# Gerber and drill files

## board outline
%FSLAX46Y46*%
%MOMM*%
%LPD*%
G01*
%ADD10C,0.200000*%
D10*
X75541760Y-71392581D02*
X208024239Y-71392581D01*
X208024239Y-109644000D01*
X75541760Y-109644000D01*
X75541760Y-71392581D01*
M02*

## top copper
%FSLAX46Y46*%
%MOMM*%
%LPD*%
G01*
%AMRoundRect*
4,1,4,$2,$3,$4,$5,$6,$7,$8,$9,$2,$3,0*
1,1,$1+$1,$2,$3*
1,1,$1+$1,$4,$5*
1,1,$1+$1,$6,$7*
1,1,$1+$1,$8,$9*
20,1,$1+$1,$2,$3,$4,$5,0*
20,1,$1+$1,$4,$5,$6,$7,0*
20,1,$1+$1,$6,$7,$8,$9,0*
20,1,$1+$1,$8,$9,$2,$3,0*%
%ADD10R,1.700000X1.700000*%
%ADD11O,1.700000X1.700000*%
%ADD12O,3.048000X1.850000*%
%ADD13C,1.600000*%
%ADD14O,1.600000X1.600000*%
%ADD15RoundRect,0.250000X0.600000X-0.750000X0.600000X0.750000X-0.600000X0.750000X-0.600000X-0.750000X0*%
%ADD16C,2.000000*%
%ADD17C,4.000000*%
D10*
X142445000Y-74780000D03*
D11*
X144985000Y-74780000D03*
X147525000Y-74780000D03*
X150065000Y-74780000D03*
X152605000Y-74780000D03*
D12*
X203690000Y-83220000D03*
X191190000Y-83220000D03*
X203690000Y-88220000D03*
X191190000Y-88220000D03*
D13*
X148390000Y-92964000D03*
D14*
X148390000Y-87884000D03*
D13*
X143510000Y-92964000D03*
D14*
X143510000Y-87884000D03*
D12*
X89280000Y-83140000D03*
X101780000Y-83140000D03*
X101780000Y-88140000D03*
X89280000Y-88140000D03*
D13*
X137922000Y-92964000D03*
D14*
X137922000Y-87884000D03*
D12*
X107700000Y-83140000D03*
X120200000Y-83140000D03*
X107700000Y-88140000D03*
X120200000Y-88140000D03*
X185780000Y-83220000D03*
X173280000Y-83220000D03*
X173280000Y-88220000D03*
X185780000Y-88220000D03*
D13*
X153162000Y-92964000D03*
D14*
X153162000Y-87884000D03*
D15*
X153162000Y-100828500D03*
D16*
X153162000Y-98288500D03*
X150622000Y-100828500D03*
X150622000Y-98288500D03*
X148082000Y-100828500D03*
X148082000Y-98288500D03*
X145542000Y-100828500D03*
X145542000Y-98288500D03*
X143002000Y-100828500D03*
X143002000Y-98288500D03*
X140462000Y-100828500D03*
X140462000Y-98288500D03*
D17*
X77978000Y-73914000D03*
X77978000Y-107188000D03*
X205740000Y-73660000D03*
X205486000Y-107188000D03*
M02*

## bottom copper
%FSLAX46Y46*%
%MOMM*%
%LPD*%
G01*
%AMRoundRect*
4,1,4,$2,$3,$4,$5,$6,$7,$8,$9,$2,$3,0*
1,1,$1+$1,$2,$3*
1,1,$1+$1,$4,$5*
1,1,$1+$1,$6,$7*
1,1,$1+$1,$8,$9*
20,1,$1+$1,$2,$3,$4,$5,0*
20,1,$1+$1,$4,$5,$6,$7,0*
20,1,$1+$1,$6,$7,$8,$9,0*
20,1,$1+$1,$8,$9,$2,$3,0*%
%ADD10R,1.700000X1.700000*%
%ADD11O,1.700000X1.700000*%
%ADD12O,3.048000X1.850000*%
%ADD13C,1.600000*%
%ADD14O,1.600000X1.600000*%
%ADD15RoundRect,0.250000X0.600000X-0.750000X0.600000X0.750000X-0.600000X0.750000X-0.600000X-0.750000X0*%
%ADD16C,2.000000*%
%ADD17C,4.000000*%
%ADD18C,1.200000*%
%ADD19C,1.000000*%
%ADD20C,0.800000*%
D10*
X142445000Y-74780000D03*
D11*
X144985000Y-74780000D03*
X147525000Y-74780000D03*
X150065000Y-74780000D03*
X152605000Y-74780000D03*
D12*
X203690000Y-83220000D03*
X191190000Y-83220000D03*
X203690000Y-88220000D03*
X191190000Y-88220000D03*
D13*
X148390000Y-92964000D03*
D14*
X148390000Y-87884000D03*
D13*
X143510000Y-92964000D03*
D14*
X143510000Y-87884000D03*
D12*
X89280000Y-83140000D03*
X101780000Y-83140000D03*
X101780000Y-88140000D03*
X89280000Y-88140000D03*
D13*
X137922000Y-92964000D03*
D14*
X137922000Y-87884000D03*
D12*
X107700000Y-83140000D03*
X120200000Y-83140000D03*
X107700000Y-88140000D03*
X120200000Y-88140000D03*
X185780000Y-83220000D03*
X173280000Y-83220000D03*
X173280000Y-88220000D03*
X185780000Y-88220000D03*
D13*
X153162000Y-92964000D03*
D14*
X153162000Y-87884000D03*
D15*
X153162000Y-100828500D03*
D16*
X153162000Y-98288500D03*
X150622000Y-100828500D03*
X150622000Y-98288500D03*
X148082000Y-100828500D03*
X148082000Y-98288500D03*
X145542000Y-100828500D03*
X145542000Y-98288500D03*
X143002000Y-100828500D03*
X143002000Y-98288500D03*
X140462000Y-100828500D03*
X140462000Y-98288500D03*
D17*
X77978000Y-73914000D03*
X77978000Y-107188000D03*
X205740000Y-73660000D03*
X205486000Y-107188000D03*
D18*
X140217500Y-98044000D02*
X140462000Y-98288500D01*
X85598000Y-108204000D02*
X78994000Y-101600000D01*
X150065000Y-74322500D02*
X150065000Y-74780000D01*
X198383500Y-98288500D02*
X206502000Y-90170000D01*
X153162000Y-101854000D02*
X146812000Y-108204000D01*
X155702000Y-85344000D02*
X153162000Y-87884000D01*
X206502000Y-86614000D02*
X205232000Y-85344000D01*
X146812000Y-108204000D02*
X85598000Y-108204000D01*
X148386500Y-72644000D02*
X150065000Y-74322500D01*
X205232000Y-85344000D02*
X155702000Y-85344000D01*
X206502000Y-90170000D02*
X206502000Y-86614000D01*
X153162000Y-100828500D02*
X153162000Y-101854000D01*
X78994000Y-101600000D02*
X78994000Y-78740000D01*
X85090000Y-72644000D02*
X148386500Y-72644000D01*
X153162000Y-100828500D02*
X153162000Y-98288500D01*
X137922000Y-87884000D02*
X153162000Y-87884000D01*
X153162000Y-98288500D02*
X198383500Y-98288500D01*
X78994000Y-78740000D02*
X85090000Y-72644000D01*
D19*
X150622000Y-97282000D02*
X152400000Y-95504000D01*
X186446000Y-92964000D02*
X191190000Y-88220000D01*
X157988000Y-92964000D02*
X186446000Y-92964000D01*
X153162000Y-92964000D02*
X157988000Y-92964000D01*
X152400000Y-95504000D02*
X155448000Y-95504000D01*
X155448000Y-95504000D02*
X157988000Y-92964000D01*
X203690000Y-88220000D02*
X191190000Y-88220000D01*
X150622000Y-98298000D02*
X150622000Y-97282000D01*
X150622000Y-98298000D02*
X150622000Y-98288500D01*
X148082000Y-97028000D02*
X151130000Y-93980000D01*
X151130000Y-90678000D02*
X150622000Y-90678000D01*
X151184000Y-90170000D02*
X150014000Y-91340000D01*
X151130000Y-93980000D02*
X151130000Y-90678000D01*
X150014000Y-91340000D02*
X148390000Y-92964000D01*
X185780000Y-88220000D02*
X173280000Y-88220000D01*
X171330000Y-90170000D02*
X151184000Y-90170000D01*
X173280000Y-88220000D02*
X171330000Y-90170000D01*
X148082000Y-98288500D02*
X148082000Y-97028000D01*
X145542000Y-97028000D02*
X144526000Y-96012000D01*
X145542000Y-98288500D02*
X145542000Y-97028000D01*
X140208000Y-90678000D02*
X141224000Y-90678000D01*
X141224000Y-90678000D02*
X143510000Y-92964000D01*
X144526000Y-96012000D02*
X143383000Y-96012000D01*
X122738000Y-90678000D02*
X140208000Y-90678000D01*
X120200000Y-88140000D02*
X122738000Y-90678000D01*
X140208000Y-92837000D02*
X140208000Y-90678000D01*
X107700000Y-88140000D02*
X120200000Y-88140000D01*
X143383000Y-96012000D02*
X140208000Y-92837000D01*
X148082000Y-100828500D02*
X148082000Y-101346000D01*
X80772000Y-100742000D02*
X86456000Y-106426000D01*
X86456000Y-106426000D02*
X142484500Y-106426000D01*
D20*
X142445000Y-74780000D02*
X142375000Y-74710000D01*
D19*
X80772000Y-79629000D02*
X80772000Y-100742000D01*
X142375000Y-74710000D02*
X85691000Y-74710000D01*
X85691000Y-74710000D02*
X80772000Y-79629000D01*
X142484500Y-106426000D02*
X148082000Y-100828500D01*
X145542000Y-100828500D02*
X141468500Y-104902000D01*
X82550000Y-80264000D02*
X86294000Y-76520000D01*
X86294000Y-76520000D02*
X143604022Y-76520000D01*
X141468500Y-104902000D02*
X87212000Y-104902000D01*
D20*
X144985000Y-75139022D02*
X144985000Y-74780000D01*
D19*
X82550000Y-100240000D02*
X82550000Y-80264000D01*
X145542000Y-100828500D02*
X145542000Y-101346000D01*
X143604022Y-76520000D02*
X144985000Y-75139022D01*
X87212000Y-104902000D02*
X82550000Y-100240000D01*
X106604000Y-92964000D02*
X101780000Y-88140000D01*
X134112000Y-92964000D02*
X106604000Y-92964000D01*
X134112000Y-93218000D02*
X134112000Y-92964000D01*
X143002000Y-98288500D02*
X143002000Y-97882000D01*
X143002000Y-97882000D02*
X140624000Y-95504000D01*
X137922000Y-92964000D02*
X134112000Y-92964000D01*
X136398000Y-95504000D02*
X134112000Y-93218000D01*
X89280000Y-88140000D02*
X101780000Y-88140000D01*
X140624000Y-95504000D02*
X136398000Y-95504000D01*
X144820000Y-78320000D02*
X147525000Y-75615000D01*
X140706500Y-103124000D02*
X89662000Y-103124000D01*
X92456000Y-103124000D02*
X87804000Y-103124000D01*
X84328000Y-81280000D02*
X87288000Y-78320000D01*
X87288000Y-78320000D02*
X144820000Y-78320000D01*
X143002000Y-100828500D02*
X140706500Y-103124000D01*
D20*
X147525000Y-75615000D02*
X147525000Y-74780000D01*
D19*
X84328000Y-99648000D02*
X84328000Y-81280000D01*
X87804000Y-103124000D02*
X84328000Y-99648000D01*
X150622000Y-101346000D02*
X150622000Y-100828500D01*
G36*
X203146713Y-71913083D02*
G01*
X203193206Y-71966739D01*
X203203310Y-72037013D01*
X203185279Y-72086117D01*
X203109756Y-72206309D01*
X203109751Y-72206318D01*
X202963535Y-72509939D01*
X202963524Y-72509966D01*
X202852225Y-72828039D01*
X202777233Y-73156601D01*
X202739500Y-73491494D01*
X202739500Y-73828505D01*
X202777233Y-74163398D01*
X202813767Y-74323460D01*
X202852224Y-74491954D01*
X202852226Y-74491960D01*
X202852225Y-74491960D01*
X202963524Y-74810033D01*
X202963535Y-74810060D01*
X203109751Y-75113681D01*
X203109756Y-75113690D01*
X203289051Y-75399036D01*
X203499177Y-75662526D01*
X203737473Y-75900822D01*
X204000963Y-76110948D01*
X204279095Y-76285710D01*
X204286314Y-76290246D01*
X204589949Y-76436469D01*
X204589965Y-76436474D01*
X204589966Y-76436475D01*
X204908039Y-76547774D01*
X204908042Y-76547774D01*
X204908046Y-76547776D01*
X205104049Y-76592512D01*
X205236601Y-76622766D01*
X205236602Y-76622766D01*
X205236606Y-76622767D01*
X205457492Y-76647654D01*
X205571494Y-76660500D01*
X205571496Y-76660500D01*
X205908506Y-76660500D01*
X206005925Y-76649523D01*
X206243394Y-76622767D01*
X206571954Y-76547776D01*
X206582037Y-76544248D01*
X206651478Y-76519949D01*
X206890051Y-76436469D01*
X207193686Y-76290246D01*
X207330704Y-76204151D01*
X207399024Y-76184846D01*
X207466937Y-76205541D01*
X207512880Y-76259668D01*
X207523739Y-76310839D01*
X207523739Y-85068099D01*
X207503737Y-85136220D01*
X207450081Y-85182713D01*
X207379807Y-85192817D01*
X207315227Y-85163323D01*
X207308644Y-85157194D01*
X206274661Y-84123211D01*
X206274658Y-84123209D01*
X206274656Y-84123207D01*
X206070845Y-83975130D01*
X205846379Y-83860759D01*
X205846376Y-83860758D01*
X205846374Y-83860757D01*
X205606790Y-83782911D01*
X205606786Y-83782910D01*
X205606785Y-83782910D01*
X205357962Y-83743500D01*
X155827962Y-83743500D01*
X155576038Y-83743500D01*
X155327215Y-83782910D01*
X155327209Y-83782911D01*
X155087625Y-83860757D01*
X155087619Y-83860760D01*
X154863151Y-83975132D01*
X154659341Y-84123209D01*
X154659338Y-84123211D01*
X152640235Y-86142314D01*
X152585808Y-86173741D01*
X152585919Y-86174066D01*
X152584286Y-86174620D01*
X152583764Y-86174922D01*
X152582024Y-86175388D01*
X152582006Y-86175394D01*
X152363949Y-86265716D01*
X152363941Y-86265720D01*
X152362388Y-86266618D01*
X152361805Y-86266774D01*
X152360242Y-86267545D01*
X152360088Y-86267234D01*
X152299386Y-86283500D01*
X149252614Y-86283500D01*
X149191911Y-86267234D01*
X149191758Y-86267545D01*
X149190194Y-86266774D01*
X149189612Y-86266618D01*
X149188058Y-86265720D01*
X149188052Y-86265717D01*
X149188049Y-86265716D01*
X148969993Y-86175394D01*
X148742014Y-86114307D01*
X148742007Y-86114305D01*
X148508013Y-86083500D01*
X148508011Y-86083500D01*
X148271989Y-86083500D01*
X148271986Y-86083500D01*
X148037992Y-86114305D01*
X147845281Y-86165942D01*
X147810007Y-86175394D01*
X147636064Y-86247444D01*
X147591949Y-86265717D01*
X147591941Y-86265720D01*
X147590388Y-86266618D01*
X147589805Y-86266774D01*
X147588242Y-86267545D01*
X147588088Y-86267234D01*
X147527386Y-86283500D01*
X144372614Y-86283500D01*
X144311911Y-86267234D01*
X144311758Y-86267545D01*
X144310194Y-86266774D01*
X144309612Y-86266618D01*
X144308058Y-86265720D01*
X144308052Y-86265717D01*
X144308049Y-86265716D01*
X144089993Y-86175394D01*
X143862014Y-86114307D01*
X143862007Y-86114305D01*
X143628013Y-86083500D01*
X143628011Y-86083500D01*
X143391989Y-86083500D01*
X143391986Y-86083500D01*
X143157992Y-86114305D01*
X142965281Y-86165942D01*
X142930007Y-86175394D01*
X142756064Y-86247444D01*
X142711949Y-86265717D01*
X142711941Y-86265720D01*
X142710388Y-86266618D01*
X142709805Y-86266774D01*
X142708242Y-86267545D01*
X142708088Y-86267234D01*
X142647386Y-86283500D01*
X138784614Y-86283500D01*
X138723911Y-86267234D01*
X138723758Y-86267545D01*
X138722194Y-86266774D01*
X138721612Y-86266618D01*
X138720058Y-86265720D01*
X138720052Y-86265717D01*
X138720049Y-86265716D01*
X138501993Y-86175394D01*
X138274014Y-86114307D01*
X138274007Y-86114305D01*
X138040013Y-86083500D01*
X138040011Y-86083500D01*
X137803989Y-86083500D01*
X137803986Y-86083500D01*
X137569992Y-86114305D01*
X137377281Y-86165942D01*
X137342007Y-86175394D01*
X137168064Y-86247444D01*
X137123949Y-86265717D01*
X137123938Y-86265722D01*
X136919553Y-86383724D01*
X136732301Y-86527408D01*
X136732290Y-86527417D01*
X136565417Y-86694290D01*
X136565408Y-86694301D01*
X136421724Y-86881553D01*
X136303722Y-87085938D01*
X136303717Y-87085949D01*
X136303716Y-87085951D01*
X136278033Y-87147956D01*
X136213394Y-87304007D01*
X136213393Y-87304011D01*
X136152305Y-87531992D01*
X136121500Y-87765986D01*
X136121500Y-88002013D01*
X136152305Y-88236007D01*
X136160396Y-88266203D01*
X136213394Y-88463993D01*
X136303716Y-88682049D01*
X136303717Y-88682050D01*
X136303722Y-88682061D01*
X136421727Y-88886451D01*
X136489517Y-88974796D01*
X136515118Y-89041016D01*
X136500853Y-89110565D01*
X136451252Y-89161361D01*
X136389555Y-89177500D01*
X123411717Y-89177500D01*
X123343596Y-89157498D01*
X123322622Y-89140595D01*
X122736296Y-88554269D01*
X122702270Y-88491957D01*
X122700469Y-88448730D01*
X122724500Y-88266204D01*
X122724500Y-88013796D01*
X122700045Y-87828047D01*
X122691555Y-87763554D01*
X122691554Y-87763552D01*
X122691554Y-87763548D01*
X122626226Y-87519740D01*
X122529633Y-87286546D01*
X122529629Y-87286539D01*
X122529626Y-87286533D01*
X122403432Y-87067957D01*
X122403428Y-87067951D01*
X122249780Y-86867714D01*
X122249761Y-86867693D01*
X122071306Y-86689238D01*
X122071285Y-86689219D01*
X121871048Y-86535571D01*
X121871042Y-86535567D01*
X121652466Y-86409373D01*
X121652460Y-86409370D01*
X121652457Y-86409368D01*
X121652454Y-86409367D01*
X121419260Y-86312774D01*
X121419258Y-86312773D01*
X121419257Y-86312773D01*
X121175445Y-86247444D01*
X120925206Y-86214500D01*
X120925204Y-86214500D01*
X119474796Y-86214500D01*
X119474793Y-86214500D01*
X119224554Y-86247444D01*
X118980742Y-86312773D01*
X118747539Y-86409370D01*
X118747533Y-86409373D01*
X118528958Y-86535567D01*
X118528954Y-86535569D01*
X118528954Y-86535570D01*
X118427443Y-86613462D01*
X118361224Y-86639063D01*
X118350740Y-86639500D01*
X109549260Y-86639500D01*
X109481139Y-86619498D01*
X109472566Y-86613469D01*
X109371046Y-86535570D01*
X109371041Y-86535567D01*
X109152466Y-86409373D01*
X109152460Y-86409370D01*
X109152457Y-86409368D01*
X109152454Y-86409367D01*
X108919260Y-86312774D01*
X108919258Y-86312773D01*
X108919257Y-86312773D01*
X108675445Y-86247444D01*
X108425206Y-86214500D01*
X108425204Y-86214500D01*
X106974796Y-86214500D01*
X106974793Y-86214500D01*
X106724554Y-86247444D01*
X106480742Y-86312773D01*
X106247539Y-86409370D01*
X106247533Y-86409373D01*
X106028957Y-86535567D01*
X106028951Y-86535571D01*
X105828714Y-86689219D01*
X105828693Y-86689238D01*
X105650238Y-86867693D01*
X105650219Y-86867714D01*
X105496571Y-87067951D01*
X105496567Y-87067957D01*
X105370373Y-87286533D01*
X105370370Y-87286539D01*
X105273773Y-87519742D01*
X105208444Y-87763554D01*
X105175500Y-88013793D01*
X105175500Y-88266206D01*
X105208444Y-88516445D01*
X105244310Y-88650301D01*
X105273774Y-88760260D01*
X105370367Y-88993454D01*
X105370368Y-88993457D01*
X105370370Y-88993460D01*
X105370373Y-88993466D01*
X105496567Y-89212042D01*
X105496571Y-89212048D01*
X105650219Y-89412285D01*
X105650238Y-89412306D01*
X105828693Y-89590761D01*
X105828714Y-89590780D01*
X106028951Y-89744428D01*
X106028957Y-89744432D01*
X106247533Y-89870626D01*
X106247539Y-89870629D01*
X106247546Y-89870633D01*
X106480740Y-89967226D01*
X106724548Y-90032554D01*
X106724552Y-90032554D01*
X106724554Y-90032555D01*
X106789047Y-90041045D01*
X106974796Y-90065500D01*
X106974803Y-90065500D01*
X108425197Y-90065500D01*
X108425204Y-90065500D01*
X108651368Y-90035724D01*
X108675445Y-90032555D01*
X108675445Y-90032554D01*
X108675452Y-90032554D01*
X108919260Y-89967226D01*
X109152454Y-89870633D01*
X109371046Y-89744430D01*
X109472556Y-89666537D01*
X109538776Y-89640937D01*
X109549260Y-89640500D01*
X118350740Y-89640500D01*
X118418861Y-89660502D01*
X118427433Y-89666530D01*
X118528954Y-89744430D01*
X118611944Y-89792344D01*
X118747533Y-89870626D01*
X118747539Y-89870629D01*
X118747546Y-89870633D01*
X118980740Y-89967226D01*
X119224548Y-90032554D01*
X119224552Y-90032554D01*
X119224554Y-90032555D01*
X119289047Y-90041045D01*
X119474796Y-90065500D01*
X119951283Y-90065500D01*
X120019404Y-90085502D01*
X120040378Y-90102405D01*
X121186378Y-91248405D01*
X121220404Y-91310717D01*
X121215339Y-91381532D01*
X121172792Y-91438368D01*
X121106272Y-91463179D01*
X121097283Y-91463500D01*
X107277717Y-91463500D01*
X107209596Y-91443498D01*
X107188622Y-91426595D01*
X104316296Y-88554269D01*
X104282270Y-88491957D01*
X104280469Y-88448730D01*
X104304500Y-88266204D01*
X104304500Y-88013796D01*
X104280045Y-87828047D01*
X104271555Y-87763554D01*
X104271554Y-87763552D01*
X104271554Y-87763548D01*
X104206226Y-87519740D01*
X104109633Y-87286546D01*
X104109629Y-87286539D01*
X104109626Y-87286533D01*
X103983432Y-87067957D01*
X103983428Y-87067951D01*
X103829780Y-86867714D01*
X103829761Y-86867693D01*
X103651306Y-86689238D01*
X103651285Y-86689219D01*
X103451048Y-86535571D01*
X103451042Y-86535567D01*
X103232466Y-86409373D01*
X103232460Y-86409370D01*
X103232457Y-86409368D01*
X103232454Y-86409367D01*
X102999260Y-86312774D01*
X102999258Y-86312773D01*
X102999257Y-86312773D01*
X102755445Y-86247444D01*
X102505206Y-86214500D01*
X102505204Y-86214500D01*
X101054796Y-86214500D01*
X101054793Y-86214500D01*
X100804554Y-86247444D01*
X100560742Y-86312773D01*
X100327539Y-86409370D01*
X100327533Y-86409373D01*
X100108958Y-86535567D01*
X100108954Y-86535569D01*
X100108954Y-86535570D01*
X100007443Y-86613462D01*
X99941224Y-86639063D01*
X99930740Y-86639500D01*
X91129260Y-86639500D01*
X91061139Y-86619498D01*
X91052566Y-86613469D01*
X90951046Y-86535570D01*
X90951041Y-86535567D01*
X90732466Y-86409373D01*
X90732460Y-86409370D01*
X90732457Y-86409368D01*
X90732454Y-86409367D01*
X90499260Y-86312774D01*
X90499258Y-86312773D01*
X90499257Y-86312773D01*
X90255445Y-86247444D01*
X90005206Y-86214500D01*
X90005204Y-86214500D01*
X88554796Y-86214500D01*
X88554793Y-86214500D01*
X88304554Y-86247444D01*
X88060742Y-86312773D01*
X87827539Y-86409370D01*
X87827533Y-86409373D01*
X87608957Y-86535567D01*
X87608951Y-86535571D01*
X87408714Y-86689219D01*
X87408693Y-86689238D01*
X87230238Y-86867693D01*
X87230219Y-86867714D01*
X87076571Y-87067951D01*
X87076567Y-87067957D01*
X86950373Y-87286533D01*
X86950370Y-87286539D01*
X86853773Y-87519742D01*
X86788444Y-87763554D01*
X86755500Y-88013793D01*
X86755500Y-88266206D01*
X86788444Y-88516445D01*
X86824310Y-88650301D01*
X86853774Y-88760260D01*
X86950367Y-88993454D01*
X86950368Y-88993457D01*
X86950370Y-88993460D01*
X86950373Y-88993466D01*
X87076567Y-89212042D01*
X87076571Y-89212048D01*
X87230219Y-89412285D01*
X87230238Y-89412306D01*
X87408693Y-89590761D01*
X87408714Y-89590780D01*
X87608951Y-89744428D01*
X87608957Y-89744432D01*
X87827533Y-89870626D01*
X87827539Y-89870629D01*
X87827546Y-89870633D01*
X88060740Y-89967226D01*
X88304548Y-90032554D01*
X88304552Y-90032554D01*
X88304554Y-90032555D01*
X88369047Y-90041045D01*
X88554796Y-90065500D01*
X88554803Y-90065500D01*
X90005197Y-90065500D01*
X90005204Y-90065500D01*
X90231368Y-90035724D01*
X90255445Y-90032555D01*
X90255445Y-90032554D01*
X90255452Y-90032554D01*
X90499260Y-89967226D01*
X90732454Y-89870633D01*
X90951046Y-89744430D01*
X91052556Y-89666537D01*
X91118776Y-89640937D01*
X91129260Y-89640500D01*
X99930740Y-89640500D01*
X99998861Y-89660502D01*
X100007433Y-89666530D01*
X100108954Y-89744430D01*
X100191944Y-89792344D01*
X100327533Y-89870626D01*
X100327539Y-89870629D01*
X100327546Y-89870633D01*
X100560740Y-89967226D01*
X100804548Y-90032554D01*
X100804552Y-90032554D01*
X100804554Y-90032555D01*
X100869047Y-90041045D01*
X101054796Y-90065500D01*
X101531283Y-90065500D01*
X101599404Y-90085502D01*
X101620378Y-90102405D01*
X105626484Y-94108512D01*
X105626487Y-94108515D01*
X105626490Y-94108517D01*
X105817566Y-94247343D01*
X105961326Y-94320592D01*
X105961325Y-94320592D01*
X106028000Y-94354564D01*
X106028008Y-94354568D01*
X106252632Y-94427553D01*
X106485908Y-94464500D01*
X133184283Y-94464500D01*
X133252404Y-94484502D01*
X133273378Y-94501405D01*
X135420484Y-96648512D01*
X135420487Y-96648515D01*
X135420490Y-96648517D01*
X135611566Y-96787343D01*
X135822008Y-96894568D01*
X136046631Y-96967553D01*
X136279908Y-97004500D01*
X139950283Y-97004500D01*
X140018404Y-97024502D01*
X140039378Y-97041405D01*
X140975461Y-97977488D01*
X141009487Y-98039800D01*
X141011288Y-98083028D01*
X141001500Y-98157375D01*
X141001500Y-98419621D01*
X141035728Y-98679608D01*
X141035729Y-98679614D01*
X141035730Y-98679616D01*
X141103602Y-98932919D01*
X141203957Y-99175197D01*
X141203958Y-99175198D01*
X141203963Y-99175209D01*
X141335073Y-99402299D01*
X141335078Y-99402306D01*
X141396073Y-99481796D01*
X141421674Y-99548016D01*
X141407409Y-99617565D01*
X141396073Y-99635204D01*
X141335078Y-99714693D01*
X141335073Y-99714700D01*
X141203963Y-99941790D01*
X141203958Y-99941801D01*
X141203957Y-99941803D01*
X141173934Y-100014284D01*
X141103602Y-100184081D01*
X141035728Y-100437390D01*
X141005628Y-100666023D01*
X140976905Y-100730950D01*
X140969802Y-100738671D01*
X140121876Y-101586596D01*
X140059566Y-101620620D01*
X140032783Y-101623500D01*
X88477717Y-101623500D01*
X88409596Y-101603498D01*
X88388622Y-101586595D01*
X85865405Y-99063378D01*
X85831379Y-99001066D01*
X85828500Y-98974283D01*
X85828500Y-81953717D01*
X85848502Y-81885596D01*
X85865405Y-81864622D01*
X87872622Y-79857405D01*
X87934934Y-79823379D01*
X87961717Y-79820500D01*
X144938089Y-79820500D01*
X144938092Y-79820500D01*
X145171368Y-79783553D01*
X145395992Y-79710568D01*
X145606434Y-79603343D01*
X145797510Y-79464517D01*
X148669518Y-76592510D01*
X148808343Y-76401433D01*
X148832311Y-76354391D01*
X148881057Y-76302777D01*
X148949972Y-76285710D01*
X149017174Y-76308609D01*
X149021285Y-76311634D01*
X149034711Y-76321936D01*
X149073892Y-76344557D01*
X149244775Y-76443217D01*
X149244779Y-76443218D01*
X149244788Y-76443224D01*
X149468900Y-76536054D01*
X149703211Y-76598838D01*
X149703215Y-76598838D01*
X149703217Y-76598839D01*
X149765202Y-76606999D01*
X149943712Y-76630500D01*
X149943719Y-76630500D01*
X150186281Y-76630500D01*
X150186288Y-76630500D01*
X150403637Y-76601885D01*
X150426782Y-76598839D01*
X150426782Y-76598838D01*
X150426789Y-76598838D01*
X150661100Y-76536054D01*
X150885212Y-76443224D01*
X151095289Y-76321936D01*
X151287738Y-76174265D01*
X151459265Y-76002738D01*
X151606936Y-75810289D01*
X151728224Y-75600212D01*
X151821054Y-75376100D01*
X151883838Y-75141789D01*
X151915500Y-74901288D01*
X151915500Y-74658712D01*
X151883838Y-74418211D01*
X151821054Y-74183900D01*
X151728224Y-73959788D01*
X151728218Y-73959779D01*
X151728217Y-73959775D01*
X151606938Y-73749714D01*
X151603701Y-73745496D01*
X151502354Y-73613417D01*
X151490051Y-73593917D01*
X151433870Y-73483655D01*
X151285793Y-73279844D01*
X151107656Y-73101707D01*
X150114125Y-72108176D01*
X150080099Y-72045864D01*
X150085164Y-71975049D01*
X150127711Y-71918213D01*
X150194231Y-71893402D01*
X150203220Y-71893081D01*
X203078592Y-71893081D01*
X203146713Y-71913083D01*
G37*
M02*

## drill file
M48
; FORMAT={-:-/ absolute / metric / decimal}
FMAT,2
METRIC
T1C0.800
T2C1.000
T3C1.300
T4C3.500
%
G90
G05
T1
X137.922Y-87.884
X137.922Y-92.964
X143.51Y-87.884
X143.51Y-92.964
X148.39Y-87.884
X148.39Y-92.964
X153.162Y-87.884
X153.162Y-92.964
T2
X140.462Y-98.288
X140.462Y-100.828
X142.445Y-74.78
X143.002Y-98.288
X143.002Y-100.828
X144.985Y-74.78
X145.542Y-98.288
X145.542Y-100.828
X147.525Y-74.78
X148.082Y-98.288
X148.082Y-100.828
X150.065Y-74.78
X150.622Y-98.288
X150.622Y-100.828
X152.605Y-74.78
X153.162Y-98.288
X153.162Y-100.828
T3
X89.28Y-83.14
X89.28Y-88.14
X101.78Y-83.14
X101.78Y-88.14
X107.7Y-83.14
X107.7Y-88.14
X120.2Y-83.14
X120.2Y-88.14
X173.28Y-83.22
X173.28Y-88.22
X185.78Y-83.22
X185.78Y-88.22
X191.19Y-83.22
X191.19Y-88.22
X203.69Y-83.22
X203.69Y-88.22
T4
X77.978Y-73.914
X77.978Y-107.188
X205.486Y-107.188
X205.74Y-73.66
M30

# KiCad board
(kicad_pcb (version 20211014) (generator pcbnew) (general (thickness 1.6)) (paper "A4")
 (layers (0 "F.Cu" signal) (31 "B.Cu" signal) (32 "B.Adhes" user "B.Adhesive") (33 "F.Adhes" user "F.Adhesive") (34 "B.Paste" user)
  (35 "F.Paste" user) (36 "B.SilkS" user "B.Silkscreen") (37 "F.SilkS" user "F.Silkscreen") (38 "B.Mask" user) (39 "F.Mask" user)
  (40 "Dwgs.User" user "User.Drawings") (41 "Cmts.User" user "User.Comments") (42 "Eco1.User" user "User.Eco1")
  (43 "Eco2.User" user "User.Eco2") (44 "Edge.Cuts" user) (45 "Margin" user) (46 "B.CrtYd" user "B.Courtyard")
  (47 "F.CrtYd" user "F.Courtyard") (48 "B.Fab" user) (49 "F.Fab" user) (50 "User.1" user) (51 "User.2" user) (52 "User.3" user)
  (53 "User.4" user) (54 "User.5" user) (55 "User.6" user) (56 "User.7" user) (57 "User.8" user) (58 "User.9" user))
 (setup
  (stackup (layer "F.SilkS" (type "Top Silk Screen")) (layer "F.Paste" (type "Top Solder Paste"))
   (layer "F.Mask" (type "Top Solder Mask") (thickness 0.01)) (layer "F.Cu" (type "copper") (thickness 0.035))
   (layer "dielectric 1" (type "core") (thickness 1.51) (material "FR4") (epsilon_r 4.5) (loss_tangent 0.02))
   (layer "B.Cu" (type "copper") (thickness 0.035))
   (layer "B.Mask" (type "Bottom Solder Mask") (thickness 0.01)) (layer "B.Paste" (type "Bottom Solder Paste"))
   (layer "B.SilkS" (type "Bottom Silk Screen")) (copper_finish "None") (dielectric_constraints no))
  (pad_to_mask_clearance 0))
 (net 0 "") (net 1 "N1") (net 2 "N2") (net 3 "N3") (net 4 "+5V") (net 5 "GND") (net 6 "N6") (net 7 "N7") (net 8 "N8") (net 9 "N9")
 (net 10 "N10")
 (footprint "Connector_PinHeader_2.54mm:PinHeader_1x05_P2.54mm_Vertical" (layer "F.Cu") (at 142.445 74.78 90)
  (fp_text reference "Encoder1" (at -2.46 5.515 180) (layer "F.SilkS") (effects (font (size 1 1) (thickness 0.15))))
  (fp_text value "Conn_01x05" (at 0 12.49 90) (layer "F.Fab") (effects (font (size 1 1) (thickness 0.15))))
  (pad "1" thru_hole rect (at 0 0 90) (size 1.7 1.7) (drill 1) (layers *.Cu *.Mask) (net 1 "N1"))
  (pad "2" thru_hole oval (at 0 2.54 90) (size 1.7 1.7) (drill 1) (layers *.Cu *.Mask) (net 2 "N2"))
  (pad "3" thru_hole oval (at 0 5.08 90) (size 1.7 1.7) (drill 1) (layers *.Cu *.Mask) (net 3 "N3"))
  (pad "4" thru_hole oval (at 0 7.62 90) (size 1.7 1.7) (drill 1) (layers *.Cu *.Mask) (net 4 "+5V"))
  (pad "5" thru_hole oval (at 0 10.16 90) (size 1.7 1.7) (drill 1) (layers *.Cu *.Mask) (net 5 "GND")))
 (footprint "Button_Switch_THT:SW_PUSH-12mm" (layer "F.Cu") (at 191.19 83.22)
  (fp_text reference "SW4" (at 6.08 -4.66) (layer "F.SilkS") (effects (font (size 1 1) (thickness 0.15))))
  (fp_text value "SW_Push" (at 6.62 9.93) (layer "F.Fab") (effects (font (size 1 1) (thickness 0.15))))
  (pad "1" thru_hole oval (at 12.5 0) (size 3.048 1.85) (drill 1.3) (layers *.Cu *.Mask) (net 5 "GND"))
  (pad "1" thru_hole oval (at 0 0) (size 3.048 1.85) (drill 1.3) (layers *.Cu *.Mask) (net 5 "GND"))
  (pad "2" thru_hole oval (at 12.5 5) (size 3.048 1.85) (drill 1.3) (layers *.Cu *.Mask) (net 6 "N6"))
  (pad "2" thru_hole oval (at 0 5) (size 3.048 1.85) (drill 1.3) (layers *.Cu *.Mask) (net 6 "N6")))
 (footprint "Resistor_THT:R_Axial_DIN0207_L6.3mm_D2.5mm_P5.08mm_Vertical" (layer "F.Cu") (at 148.39 92.964 90)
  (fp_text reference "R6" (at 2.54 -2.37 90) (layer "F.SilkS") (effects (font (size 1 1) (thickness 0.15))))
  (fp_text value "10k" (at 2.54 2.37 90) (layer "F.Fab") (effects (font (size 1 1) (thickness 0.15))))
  (pad "1" thru_hole circle (at 0 0 90) (size 1.6 1.6) (drill 0.8) (layers *.Cu *.Mask) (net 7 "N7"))
  (pad "2" thru_hole oval (at 5.08 0 90) (size 1.6 1.6) (drill 0.8) (layers *.Cu *.Mask) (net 4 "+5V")))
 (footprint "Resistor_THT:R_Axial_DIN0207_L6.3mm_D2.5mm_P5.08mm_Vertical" (layer "F.Cu") (at 143.51 92.964 90)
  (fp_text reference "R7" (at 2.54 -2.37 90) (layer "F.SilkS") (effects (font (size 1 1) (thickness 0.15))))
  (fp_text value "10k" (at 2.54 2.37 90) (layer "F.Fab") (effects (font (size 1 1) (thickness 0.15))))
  (pad "1" thru_hole circle (at 0 0 90) (size 1.6 1.6) (drill 0.8) (layers *.Cu *.Mask) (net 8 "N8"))
  (pad "2" thru_hole oval (at 5.08 0 90) (size 1.6 1.6) (drill 0.8) (layers *.Cu *.Mask) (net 4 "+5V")))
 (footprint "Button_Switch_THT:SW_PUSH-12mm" (layer "F.Cu") (at 89.28 83.14)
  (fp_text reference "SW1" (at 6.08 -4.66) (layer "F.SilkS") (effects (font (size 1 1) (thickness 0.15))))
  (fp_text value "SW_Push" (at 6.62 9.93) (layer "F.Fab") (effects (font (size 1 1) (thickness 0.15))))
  (pad "1" thru_hole oval (at 0 0) (size 3.048 1.85) (drill 1.3) (layers *.Cu *.Mask) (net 5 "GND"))
  (pad "1" thru_hole oval (at 12.5 0) (size 3.048 1.85) (drill 1.3) (layers *.Cu *.Mask) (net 5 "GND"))
  (pad "2" thru_hole oval (at 12.5 5) (size 3.048 1.85) (drill 1.3) (layers *.Cu *.Mask) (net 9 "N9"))
  (pad "2" thru_hole oval (at 0 5) (size 3.048 1.85) (drill 1.3) (layers *.Cu *.Mask) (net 9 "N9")))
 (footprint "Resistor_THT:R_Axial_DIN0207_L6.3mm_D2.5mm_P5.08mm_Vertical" (layer "F.Cu") (at 137.922 92.964 90)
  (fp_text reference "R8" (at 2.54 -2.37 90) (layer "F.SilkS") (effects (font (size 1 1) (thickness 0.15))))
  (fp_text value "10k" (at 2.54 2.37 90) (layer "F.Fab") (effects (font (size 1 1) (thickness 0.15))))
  (pad "1" thru_hole circle (at 0 0 90) (size 1.6 1.6) (drill 0.8) (layers *.Cu *.Mask) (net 9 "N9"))
  (pad "2" thru_hole oval (at 5.08 0 90) (size 1.6 1.6) (drill 0.8) (layers *.Cu *.Mask) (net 4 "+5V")))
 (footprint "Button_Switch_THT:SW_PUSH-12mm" (layer "F.Cu") (at 107.7 83.14)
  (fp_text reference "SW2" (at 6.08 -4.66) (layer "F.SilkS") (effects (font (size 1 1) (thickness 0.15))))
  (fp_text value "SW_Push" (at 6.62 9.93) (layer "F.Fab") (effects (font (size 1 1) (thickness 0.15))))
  (pad "1" thru_hole oval (at 0 0) (size 3.048 1.85) (drill 1.3) (layers *.Cu *.Mask) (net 5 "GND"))
  (pad "1" thru_hole oval (at 12.5 0) (size 3.048 1.85) (drill 1.3) (layers *.Cu *.Mask) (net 5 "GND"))
  (pad "2" thru_hole oval (at 0 5) (size 3.048 1.85) (drill 1.3) (layers *.Cu *.Mask) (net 8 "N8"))
  (pad "2" thru_hole oval (at 12.5 5) (size 3.048 1.85) (drill 1.3) (layers *.Cu *.Mask) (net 8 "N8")))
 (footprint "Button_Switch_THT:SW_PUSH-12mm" (layer "F.Cu") (at 173.28 83.22)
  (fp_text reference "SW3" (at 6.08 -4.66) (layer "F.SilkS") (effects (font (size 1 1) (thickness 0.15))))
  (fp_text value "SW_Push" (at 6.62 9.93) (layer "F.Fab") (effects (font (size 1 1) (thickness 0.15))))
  (pad "1" thru_hole oval (at 12.5 0) (size 3.048 1.85) (drill 1.3) (layers *.Cu *.Mask) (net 5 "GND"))
  (pad "1" thru_hole oval (at 0 0) (size 3.048 1.85) (drill 1.3) (layers *.Cu *.Mask) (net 5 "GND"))
  (pad "2" thru_hole oval (at 0 5) (size 3.048 1.85) (drill 1.3) (layers *.Cu *.Mask) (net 7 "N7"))
  (pad "2" thru_hole oval (at 12.5 5) (size 3.048 1.85) (drill 1.3) (layers *.Cu *.Mask) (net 7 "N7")))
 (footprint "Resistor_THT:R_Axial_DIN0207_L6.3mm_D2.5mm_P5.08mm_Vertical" (layer "F.Cu") (at 153.162 92.964 90)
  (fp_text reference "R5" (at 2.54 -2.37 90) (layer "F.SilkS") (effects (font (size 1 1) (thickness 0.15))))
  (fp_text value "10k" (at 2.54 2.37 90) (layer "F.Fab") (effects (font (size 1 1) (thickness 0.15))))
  (pad "1" thru_hole circle (at 0 0 90) (size 1.6 1.6) (drill 0.8) (layers *.Cu *.Mask) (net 6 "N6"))
  (pad "2" thru_hole oval (at 5.08 0 90) (size 1.6 1.6) (drill 0.8) (layers *.Cu *.Mask) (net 4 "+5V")))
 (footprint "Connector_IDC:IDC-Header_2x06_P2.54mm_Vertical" (layer "B.Cu") (at 153.162 100.8285 90)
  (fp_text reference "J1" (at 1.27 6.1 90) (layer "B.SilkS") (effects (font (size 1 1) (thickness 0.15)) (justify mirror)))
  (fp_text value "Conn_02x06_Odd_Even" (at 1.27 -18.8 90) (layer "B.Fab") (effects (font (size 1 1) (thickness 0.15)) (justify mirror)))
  (pad "1" thru_hole roundrect (at 0 0 90) (size 2 1.7) (drill 1) (layers *.Cu *.Mask) (roundrect_rratio 0.147059) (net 4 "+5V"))
  (pad "2" thru_hole circle (at 2.54 0 90) (size 2 2) (drill 1) (layers *.Cu *.Mask) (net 4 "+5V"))
  (pad "3" thru_hole circle (at 0 -2.54 90) (size 2 2) (drill 1) (layers *.Cu *.Mask) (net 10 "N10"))
  (pad "4" thru_hole circle (at 2.54 -2.54 90) (size 2 2) (drill 1) (layers *.Cu *.Mask) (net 6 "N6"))
  (pad "5" thru_hole circle (at 0 -5.08 90) (size 2 2) (drill 1) (layers *.Cu *.Mask) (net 1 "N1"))
  (pad "6" thru_hole circle (at 2.54 -5.08 90) (size 2 2) (drill 1) (layers *.Cu *.Mask) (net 7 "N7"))
  (pad "7" thru_hole circle (at 0 -7.62 90) (size 2 2) (drill 1) (layers *.Cu *.Mask) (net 2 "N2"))
  (pad "8" thru_hole circle (at 2.54 -7.62 90) (size 2 2) (drill 1) (layers *.Cu *.Mask) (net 8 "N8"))
  (pad "9" thru_hole circle (at 0 -10.16 90) (size 2 2) (drill 1) (layers *.Cu *.Mask) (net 3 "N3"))
  (pad "10" thru_hole circle (at 2.54 -10.16 90) (size 2 2) (drill 1) (layers *.Cu *.Mask) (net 9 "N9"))
  (pad "11" thru_hole circle (at 0 -12.7 90) (size 2 2) (drill 1) (layers *.Cu *.Mask) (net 5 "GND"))
  (pad "12" thru_hole circle (at 2.54 -12.7 90) (size 2 2) (drill 1) (layers *.Cu *.Mask) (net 5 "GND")))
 (gr_rect (start 75.54176 71.392581) (end 208.024239 109.644) (layer "Edge.Cuts") (width 0.2) (fill none))
 (via (at 77.978 73.914) (size 4) (drill 3.5) (layers "F.Cu" "B.Cu") (free) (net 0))
 (via (at 77.978 107.188) (size 4) (drill 3.5) (layers "F.Cu" "B.Cu") (free) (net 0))
 (via (at 205.74 73.66) (size 4) (drill 3.5) (layers "F.Cu" "B.Cu") (free) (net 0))
 (via (at 205.486 107.188) (size 4) (drill 3.5) (layers "F.Cu" "B.Cu") (free) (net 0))
 (segment (start 140.2175 98.044) (end 140.462 98.2885) (width 1.2) (layer "B.Cu") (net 5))
 (segment (start 85.598 108.204) (end 78.994 101.6) (width 1.2) (layer "B.Cu") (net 4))
 (segment (start 150.065 74.3225) (end 150.065 74.78) (width 1.2) (layer "B.Cu") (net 4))
 (segment (start 198.3835 98.2885) (end 206.502 90.17) (width 1.2) (layer "B.Cu") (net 4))
 (segment (start 153.162 101.854) (end 146.812 108.204) (width 1.2) (layer "B.Cu") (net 4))
 (segment (start 155.702 85.344) (end 153.162 87.884) (width 1.2) (layer "B.Cu") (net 4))
 (segment (start 206.502 86.614) (end 205.232 85.344) (width 1.2) (layer "B.Cu") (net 4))
 (segment (start 146.812 108.204) (end 85.598 108.204) (width 1.2) (layer "B.Cu") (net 4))
 (segment (start 148.3865 72.644) (end 150.065 74.3225) (width 1.2) (layer "B.Cu") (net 4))
 (segment (start 205.232 85.344) (end 155.702 85.344) (width 1.2) (layer "B.Cu") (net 4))
 (segment (start 206.502 90.17) (end 206.502 86.614) (width 1.2) (layer "B.Cu") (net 4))
 (segment (start 153.162 100.8285) (end 153.162 101.854) (width 1.2) (layer "B.Cu") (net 4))
 (segment (start 78.994 101.6) (end 78.994 78.74) (width 1.2) (layer "B.Cu") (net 4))
 (segment (start 85.09 72.644) (end 148.3865 72.644) (width 1.2) (layer "B.Cu") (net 4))
 (segment (start 153.162 100.8285) (end 153.162 98.2885) (width 1.2) (layer "B.Cu") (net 4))
 (segment (start 137.922 87.884) (end 153.162 87.884) (width 1.2) (layer "B.Cu") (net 4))
 (segment (start 153.162 98.2885) (end 198.3835 98.2885) (width 1.2) (layer "B.Cu") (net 4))
 (segment (start 78.994 78.74) (end 85.09 72.644) (width 1.2) (layer "B.Cu") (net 4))
 (segment (start 150.622 97.282) (end 152.4 95.504) (width 1) (layer "B.Cu") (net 6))
 (segment (start 186.446 92.964) (end 191.19 88.22) (width 1) (layer "B.Cu") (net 6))
 (segment (start 157.988 92.964) (end 186.446 92.964) (width 1) (layer "B.Cu") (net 6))
 (segment (start 153.162 92.964) (end 157.988 92.964) (width 1) (layer "B.Cu") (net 6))
 (segment (start 152.4 95.504) (end 155.448 95.504) (width 1) (layer "B.Cu") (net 6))
 (segment (start 155.448 95.504) (end 157.988 92.964) (width 1) (layer "B.Cu") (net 6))
 (segment (start 203.69 88.22) (end 191.19 88.22) (width 1) (layer "B.Cu") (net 6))
 (segment (start 150.622 98.298) (end 150.622 97.282) (width 1) (layer "B.Cu") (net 6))
 (segment (start 150.622 98.298) (end 150.622 98.2885) (width 1) (layer "B.Cu") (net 6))
 (segment (start 148.082 97.028) (end 151.13 93.98) (width 1) (layer "B.Cu") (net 7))
 (segment (start 151.13 90.678) (end 150.622 90.678) (width 1) (layer "B.Cu") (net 7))
 (segment (start 151.184 90.17) (end 150.014 91.34) (width 1) (layer "B.Cu") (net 7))
 (segment (start 151.13 93.98) (end 151.13 90.678) (width 1) (layer "B.Cu") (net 7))
 (segment (start 150.014 91.34) (end 148.39 92.964) (width 1) (layer "B.Cu") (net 7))
 (segment (start 185.78 88.22) (end 173.28 88.22) (width 1) (layer "B.Cu") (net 7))
 (segment (start 171.33 90.17) (end 151.184 90.17) (width 1) (layer "B.Cu") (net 7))
 (segment (start 173.28 88.22) (end 171.33 90.17) (width 1) (layer "B.Cu") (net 7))
 (segment (start 148.082 98.2885) (end 148.082 97.028) (width 1) (layer "B.Cu") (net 7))
 (segment (start 145.542 97.028) (end 144.526 96.012) (width 1) (layer "B.Cu") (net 8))
 (segment (start 145.542 98.2885) (end 145.542 97.028) (width 1) (layer "B.Cu") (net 8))
 (segment (start 140.208 90.678) (end 141.224 90.678) (width 1) (layer "B.Cu") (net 8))
 (segment (start 141.224 90.678) (end 143.51 92.964) (width 1) (layer "B.Cu") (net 8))
 (segment (start 144.526 96.012) (end 143.383 96.012) (width 1) (layer "B.Cu") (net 8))
 (segment (start 122.738 90.678) (end 140.208 90.678) (width 1) (layer "B.Cu") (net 8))
 (segment (start 120.2 88.14) (end 122.738 90.678) (width 1) (layer "B.Cu") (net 8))
 (segment (start 140.208 92.837) (end 140.208 90.678) (width 1) (layer "B.Cu") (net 8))
 (segment (start 107.7 88.14) (end 120.2 88.14) (width 1) (layer "B.Cu") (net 8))
 (segment (start 143.383 96.012) (end 140.208 92.837) (width 1) (layer "B.Cu") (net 8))
 (segment (start 148.082 100.8285) (end 148.082 101.346) (width 1) (layer "B.Cu") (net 1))
 (segment (start 80.772 100.742) (end 86.456 106.426) (width 1) (layer "B.Cu") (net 1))
 (segment (start 86.456 106.426) (end 142.4845 106.426) (width 1) (layer "B.Cu") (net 1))
 (segment (start 142.445 74.78) (end 142.375 74.71) (width 0.8) (layer "B.Cu") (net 1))
 (segment (start 80.772 79.629) (end 80.772 100.742) (width 1) (layer "B.Cu") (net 1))
 (segment (start 142.375 74.71) (end 85.691 74.71) (width 1) (layer "B.Cu") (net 1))
 (segment (start 85.691 74.71) (end 80.772 79.629) (width 1) (layer "B.Cu") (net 1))
 (segment (start 142.4845 106.426) (end 148.082 100.8285) (width 1) (layer "B.Cu") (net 1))
 (segment (start 145.542 100.8285) (end 141.4685 104.902) (width 1) (layer "B.Cu") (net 2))
 (segment (start 82.55 80.264) (end 86.294 76.52) (width 1) (layer "B.Cu") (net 2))
 (segment (start 86.294 76.52) (end 143.604022 76.52) (width 1) (layer "B.Cu") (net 2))
 (segment (start 141.4685 104.902) (end 87.212 104.902) (width 1) (layer "B.Cu") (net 2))
 (segment (start 144.985 75.139022) (end 144.985 74.78) (width 0.8) (layer "B.Cu") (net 2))
 (segment (start 82.55 100.24) (end 82.55 80.264) (width 1) (layer "B.Cu") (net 2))
 (segment (start 145.542 100.8285) (end 145.542 101.346) (width 1) (layer "B.Cu") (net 2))
 (segment (start 143.604022 76.52) (end 144.985 75.139022) (width 1) (layer "B.Cu") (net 2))
 (segment (start 87.212 104.902) (end 82.55 100.24) (width 1) (layer "B.Cu") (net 2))
 (segment (start 106.604 92.964) (end 101.78 88.14) (width 1) (layer "B.Cu") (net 9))
 (segment (start 134.112 92.964) (end 106.604 92.964) (width 1) (layer "B.Cu") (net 9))
 (segment (start 134.112 93.218) (end 134.112 92.964) (width 1) (layer "B.Cu") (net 9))
 (segment (start 143.002 98.2885) (end 143.002 97.882) (width 1) (layer "B.Cu") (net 9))
 (segment (start 143.002 97.882) (end 140.624 95.504) (width 1) (layer "B.Cu") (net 9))
 (segment (start 137.922 92.964) (end 134.112 92.964) (width 1) (layer "B.Cu") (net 9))
 (segment (start 136.398 95.504) (end 134.112 93.218) (width 1) (layer "B.Cu") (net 9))
 (segment (start 89.28 88.14) (end 101.78 88.14) (width 1) (layer "B.Cu") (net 9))
 (segment (start 140.624 95.504) (end 136.398 95.504) (width 1) (layer "B.Cu") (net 9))
 (segment (start 144.82 78.32) (end 147.525 75.615) (width 1) (layer "B.Cu") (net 3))
 (segment (start 140.7065 103.124) (end 89.662 103.124) (width 1) (layer "B.Cu") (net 3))
 (segment (start 92.456 103.124) (end 87.804 103.124) (width 1) (layer "B.Cu") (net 3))
 (segment (start 84.328 81.28) (end 87.288 78.32) (width 1) (layer "B.Cu") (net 3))
 (segment (start 87.288 78.32) (end 144.82 78.32) (width 1) (layer "B.Cu") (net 3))
 (segment (start 143.002 100.8285) (end 140.7065 103.124) (width 1) (layer "B.Cu") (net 3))
 (segment (start 147.525 75.615) (end 147.525 74.78) (width 0.8) (layer "B.Cu") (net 3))
 (segment (start 84.328 99.648) (end 84.328 81.28) (width 1) (layer "B.Cu") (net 3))
 (segment (start 87.804 103.124) (end 84.328 99.648) (width 1) (layer "B.Cu") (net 3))
 (segment (start 150.622 101.346) (end 150.622 100.8285) (width 1) (layer "B.Cu") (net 10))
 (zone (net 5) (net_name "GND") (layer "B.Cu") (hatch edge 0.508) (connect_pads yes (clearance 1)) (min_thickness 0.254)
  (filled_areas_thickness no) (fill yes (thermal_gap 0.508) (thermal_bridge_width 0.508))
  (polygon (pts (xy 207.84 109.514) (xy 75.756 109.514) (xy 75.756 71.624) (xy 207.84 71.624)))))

